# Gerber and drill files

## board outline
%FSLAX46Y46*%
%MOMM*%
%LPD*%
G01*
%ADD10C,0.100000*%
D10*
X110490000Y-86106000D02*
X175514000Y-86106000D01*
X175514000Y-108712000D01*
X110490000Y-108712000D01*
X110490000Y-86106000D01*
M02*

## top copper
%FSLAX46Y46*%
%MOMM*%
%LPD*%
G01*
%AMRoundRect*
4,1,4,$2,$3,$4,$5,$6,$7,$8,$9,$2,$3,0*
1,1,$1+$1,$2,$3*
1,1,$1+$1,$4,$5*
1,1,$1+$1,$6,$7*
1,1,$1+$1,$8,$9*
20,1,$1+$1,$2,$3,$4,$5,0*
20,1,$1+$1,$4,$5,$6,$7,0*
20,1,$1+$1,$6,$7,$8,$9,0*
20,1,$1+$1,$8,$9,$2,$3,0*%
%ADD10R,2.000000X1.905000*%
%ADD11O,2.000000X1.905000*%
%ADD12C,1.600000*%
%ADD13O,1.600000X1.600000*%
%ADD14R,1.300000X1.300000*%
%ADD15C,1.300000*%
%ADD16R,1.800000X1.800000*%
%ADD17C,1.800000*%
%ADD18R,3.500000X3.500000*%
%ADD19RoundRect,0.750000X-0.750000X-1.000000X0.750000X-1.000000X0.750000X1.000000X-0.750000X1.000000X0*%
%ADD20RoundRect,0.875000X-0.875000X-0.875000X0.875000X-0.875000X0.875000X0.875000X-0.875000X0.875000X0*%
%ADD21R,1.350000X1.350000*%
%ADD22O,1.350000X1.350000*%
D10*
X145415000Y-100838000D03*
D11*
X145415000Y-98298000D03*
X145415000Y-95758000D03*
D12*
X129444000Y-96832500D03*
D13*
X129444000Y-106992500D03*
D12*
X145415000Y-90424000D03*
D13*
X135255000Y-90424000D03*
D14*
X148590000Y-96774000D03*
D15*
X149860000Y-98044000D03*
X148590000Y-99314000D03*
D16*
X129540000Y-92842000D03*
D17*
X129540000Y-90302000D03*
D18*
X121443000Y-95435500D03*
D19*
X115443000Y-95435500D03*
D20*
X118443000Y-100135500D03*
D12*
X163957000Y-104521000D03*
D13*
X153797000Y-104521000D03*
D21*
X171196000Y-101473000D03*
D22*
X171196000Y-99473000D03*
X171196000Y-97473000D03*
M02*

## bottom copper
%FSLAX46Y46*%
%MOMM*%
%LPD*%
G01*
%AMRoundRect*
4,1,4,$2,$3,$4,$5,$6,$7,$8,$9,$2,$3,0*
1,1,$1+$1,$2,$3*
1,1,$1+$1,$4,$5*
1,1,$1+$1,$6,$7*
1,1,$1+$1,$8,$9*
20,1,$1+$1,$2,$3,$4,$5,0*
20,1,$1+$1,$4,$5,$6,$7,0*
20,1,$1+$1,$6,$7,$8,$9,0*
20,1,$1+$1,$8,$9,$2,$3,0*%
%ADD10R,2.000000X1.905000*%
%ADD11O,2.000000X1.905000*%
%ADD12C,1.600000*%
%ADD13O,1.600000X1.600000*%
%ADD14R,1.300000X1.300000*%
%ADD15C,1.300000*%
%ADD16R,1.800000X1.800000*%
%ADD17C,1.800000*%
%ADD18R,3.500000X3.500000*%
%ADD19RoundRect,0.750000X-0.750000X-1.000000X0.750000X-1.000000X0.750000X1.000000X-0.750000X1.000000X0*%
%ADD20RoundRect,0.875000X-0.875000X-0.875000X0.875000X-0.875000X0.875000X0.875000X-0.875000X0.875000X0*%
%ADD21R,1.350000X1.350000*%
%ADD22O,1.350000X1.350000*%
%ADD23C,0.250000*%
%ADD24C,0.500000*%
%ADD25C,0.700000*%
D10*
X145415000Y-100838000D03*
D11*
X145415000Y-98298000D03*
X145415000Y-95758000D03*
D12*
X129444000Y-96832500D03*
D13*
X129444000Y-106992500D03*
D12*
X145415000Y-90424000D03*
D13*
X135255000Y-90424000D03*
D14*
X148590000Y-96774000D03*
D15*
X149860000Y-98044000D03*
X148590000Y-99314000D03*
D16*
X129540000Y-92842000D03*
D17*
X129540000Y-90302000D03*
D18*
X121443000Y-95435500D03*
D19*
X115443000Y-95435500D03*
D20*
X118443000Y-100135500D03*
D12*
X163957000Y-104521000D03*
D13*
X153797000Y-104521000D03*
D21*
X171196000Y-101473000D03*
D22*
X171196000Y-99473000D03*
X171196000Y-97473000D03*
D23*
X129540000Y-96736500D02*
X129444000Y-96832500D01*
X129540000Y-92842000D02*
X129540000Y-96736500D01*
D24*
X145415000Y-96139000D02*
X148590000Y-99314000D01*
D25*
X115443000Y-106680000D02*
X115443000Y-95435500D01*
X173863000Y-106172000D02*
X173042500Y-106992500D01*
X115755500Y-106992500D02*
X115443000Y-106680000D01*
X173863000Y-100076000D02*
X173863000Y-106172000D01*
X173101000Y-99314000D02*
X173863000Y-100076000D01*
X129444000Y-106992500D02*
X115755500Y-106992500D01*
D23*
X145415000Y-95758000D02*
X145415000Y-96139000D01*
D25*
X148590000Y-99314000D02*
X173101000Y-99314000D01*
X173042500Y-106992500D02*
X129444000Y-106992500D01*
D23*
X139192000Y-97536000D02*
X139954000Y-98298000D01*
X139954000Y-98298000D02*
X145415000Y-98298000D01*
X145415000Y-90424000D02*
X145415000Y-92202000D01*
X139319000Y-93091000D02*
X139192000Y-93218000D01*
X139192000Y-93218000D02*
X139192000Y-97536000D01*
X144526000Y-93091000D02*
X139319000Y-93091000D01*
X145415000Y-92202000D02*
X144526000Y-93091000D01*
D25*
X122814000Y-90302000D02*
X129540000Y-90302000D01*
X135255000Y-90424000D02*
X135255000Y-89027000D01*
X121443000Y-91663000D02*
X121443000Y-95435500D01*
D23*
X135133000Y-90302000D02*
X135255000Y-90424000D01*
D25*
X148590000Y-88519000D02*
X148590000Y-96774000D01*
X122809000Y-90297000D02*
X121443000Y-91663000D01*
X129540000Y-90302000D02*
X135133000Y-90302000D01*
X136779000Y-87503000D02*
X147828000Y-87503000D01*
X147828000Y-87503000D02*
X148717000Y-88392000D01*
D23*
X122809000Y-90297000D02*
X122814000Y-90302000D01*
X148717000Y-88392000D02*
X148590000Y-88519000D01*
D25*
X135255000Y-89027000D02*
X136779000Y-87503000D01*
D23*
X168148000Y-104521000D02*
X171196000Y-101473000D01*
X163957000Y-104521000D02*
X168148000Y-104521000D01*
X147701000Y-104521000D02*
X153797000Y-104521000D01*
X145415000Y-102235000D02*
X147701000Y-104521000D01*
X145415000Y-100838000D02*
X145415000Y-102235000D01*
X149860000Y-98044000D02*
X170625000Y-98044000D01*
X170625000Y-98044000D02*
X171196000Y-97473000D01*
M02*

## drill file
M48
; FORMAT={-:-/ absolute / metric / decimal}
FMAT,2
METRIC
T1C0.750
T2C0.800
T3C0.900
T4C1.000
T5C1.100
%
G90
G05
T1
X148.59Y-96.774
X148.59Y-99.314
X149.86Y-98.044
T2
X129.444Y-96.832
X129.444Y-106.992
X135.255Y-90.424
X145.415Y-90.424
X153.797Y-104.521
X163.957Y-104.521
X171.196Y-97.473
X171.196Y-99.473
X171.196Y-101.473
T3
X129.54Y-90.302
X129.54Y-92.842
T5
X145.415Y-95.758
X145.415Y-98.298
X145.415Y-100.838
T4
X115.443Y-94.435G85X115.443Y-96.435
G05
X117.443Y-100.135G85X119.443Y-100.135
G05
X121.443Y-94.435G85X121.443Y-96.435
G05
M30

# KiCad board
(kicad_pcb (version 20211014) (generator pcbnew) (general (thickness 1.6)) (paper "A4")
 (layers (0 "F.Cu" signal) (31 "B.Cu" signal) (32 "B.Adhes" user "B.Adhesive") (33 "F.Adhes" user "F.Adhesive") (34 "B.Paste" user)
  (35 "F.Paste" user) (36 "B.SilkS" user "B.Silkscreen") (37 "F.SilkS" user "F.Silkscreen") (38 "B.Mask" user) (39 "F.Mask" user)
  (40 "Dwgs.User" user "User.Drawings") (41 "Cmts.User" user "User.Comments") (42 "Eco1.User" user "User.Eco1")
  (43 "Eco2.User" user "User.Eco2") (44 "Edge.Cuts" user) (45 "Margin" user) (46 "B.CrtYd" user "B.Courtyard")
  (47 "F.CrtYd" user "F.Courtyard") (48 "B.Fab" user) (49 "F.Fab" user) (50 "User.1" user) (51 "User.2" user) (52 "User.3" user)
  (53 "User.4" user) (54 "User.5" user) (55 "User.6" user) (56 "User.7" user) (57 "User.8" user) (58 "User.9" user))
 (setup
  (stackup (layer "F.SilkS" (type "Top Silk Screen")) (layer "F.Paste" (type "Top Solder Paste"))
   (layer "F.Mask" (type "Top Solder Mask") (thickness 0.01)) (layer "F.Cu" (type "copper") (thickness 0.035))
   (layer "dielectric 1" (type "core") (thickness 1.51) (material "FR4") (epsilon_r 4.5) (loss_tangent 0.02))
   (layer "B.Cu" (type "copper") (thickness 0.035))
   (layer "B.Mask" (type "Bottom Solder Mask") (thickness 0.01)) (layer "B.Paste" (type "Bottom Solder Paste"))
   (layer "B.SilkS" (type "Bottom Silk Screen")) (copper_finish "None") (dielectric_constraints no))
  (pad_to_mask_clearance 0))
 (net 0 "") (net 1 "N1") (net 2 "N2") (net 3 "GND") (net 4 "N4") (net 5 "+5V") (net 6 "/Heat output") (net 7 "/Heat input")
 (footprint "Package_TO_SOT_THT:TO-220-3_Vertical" (layer "F.Cu") (at 145.415 100.838 90)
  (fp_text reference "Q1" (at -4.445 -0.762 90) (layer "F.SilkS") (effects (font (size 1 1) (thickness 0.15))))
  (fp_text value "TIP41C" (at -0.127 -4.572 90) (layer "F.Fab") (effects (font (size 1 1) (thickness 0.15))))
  (pad "1" thru_hole rect (at 0 0 90) (size 1.905 2) (drill 1.1) (layers *.Cu *.Mask) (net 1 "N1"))
  (pad "2" thru_hole oval (at 2.54 0 90) (size 1.905 2) (drill 1.1) (layers *.Cu *.Mask) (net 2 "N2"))
  (pad "3" thru_hole oval (at 5.08 0 90) (size 1.905 2) (drill 1.1) (layers *.Cu *.Mask) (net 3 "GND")))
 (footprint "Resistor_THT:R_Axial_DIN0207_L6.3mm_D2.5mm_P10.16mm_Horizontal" (layer "F.Cu") (at 129.444 96.8325 -90)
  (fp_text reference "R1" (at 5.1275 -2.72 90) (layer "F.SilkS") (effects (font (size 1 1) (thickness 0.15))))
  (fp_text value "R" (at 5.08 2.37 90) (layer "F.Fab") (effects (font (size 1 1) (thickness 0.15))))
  (pad "1" thru_hole circle (at 0 0 270) (size 1.6 1.6) (drill 0.8) (layers *.Cu *.Mask) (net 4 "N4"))
  (pad "2" thru_hole oval (at 10.16 0 270) (size 1.6 1.6) (drill 0.8) (layers *.Cu *.Mask) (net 3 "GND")))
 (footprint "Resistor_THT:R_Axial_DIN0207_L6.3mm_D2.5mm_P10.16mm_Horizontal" (layer "F.Cu") (at 145.415 90.424 180)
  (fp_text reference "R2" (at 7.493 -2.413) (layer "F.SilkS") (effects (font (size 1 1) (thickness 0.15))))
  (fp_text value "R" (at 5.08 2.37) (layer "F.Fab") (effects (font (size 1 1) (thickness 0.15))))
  (pad "1" thru_hole circle (at 0 0 180) (size 1.6 1.6) (drill 0.8) (layers *.Cu *.Mask) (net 2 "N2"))
  (pad "2" thru_hole oval (at 10.16 0 180) (size 1.6 1.6) (drill 0.8) (layers *.Cu *.Mask) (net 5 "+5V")))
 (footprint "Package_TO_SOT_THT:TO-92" (layer "F.Cu") (at 148.59 96.774 -90)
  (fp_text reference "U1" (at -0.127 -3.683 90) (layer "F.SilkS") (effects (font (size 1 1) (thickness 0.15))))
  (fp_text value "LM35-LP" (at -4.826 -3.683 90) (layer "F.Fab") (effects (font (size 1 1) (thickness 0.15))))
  (pad "1" thru_hole rect (at 0 0 270) (size 1.3 1.3) (drill 0.75) (layers *.Cu *.Mask) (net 5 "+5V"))
  (pad "2" thru_hole circle (at 1.27 -1.27 270) (size 1.3 1.3) (drill 0.75) (layers *.Cu *.Mask) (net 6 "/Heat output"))
  (pad "3" thru_hole circle (at 2.54 0 270) (size 1.3 1.3) (drill 0.75) (layers *.Cu *.Mask) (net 3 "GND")))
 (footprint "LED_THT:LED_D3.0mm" (layer "F.Cu") (at 129.54 92.842 90)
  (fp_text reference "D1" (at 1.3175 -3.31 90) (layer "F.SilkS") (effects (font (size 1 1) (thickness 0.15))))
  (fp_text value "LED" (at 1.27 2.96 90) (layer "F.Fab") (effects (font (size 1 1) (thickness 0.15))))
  (pad "1" thru_hole rect (at 0 0 90) (size 1.8 1.8) (drill 0.9) (layers *.Cu *.Mask) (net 4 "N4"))
  (pad "2" thru_hole circle (at 2.54 0 90) (size 1.8 1.8) (drill 0.9) (layers *.Cu *.Mask) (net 5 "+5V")))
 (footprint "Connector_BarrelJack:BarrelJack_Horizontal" (layer "F.Cu") (at 121.443 95.4355)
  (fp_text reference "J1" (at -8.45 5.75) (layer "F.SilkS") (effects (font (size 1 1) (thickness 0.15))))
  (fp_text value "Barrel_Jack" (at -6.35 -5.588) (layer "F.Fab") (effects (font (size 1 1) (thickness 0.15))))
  (pad "1" thru_hole rect (at 0 0) (size 3.5 3.5) (drill oval 1 3) (layers *.Cu *.Mask) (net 5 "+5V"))
  (pad "2" thru_hole roundrect (at -6 0) (size 3 3.5) (drill oval 1 3) (layers *.Cu *.Mask) (roundrect_rratio 0.25) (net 3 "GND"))
  (pad "3" thru_hole roundrect (at -3 4.7) (size 3.5 3.5) (drill oval 3 1) (layers *.Cu *.Mask) (roundrect_rratio 0.25)))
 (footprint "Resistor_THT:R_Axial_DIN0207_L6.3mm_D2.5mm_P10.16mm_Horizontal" (layer "F.Cu") (at 163.957 104.521 180)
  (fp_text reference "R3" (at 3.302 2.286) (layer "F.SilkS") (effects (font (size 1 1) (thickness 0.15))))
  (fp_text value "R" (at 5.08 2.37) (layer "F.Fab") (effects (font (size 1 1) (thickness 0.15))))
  (pad "1" thru_hole circle (at 0 0 180) (size 1.6 1.6) (drill 0.8) (layers *.Cu *.Mask) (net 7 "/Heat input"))
  (pad "2" thru_hole oval (at 10.16 0 180) (size 1.6 1.6) (drill 0.8) (layers *.Cu *.Mask) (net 1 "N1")))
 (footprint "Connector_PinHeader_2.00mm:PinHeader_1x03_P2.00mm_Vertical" (layer "F.Cu") (at 171.196 101.473 180)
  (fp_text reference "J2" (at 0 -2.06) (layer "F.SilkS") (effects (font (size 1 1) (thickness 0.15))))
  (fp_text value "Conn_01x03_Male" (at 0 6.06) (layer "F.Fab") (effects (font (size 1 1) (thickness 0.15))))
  (pad "1" thru_hole rect (at 0 0 180) (size 1.35 1.35) (drill 0.8) (layers *.Cu *.Mask) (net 7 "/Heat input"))
  (pad "2" thru_hole oval (at 0 2 180) (size 1.35 1.35) (drill 0.8) (layers *.Cu *.Mask) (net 3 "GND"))
  (pad "3" thru_hole oval (at 0 4 180) (size 1.35 1.35) (drill 0.8) (layers *.Cu *.Mask) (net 6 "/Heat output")))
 (gr_rect (start 110.49 86.106) (end 175.514 108.712) (layer "Edge.Cuts") (width 0.1) (fill none))
 (segment (start 129.54 96.7365) (end 129.444 96.8325) (width 0.25) (layer "B.Cu") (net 4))
 (segment (start 129.54 92.842) (end 129.54 96.7365) (width 0.25) (layer "B.Cu") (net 4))
 (segment (start 145.415 96.139) (end 148.59 99.314) (width 0.5) (layer "B.Cu") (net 3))
 (segment (start 115.443 106.68) (end 115.443 95.4355) (width 0.7) (layer "B.Cu") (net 3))
 (segment (start 173.863 106.172) (end 173.0425 106.9925) (width 0.7) (layer "B.Cu") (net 3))
 (segment (start 115.7555 106.9925) (end 115.443 106.68) (width 0.7) (layer "B.Cu") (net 3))
 (segment (start 173.863 100.076) (end 173.863 106.172) (width 0.7) (layer "B.Cu") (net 3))
 (segment (start 173.101 99.314) (end 173.863 100.076) (width 0.7) (layer "B.Cu") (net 3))
 (segment (start 129.444 106.9925) (end 115.7555 106.9925) (width 0.7) (layer "B.Cu") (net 3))
 (segment (start 145.415 95.758) (end 145.415 96.139) (width 0.25) (layer "B.Cu") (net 3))
 (segment (start 148.59 99.314) (end 173.101 99.314) (width 0.7) (layer "B.Cu") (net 3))
 (segment (start 173.0425 106.9925) (end 129.444 106.9925) (width 0.7) (layer "B.Cu") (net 3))
 (segment (start 139.192 97.536) (end 139.954 98.298) (width 0.25) (layer "B.Cu") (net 2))
 (segment (start 139.954 98.298) (end 145.415 98.298) (width 0.25) (layer "B.Cu") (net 2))
 (segment (start 145.415 90.424) (end 145.415 92.202) (width 0.25) (layer "B.Cu") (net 2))
 (segment (start 139.319 93.091) (end 139.192 93.218) (width 0.25) (layer "B.Cu") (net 2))
 (segment (start 139.192 93.218) (end 139.192 97.536) (width 0.25) (layer "B.Cu") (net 2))
 (segment (start 144.526 93.091) (end 139.319 93.091) (width 0.25) (layer "B.Cu") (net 2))
 (segment (start 145.415 92.202) (end 144.526 93.091) (width 0.25) (layer "B.Cu") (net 2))
 (segment (start 122.814 90.302) (end 129.54 90.302) (width 0.7) (layer "B.Cu") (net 5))
 (segment (start 135.255 90.424) (end 135.255 89.027) (width 0.7) (layer "B.Cu") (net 5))
 (segment (start 121.443 91.663) (end 121.443 95.4355) (width 0.7) (layer "B.Cu") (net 5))
 (segment (start 135.133 90.302) (end 135.255 90.424) (width 0.25) (layer "B.Cu") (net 5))
 (segment (start 148.59 88.519) (end 148.59 96.774) (width 0.7) (layer "B.Cu") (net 5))
 (segment (start 122.809 90.297) (end 121.443 91.663) (width 0.7) (layer "B.Cu") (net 5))
 (segment (start 129.54 90.302) (end 135.133 90.302) (width 0.7) (layer "B.Cu") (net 5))
 (segment (start 136.779 87.503) (end 147.828 87.503) (width 0.7) (layer "B.Cu") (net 5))
 (segment (start 147.828 87.503) (end 148.717 88.392) (width 0.7) (layer "B.Cu") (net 5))
 (segment (start 122.809 90.297) (end 122.814 90.302) (width 0.25) (layer "B.Cu") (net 5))
 (segment (start 148.717 88.392) (end 148.59 88.519) (width 0.25) (layer "B.Cu") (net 5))
 (segment (start 135.255 89.027) (end 136.779 87.503) (width 0.7) (layer "B.Cu") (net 5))
 (segment (start 168.148 104.521) (end 171.196 101.473) (width 0.25) (layer "B.Cu") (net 7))
 (segment (start 163.957 104.521) (end 168.148 104.521) (width 0.25) (layer "B.Cu") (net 7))
 (segment (start 147.701 104.521) (end 153.797 104.521) (width 0.25) (layer "B.Cu") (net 1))
 (segment (start 145.415 102.235) (end 147.701 104.521) (width 0.25) (layer "B.Cu") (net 1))
 (segment (start 145.415 100.838) (end 145.415 102.235) (width 0.25) (layer "B.Cu") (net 1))
 (segment (start 149.86 98.044) (end 170.625 98.044) (width 0.25) (layer "B.Cu") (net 6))
 (segment (start 170.625 98.044) (end 171.196 97.473) (width 0.25) (layer "B.Cu") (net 6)))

